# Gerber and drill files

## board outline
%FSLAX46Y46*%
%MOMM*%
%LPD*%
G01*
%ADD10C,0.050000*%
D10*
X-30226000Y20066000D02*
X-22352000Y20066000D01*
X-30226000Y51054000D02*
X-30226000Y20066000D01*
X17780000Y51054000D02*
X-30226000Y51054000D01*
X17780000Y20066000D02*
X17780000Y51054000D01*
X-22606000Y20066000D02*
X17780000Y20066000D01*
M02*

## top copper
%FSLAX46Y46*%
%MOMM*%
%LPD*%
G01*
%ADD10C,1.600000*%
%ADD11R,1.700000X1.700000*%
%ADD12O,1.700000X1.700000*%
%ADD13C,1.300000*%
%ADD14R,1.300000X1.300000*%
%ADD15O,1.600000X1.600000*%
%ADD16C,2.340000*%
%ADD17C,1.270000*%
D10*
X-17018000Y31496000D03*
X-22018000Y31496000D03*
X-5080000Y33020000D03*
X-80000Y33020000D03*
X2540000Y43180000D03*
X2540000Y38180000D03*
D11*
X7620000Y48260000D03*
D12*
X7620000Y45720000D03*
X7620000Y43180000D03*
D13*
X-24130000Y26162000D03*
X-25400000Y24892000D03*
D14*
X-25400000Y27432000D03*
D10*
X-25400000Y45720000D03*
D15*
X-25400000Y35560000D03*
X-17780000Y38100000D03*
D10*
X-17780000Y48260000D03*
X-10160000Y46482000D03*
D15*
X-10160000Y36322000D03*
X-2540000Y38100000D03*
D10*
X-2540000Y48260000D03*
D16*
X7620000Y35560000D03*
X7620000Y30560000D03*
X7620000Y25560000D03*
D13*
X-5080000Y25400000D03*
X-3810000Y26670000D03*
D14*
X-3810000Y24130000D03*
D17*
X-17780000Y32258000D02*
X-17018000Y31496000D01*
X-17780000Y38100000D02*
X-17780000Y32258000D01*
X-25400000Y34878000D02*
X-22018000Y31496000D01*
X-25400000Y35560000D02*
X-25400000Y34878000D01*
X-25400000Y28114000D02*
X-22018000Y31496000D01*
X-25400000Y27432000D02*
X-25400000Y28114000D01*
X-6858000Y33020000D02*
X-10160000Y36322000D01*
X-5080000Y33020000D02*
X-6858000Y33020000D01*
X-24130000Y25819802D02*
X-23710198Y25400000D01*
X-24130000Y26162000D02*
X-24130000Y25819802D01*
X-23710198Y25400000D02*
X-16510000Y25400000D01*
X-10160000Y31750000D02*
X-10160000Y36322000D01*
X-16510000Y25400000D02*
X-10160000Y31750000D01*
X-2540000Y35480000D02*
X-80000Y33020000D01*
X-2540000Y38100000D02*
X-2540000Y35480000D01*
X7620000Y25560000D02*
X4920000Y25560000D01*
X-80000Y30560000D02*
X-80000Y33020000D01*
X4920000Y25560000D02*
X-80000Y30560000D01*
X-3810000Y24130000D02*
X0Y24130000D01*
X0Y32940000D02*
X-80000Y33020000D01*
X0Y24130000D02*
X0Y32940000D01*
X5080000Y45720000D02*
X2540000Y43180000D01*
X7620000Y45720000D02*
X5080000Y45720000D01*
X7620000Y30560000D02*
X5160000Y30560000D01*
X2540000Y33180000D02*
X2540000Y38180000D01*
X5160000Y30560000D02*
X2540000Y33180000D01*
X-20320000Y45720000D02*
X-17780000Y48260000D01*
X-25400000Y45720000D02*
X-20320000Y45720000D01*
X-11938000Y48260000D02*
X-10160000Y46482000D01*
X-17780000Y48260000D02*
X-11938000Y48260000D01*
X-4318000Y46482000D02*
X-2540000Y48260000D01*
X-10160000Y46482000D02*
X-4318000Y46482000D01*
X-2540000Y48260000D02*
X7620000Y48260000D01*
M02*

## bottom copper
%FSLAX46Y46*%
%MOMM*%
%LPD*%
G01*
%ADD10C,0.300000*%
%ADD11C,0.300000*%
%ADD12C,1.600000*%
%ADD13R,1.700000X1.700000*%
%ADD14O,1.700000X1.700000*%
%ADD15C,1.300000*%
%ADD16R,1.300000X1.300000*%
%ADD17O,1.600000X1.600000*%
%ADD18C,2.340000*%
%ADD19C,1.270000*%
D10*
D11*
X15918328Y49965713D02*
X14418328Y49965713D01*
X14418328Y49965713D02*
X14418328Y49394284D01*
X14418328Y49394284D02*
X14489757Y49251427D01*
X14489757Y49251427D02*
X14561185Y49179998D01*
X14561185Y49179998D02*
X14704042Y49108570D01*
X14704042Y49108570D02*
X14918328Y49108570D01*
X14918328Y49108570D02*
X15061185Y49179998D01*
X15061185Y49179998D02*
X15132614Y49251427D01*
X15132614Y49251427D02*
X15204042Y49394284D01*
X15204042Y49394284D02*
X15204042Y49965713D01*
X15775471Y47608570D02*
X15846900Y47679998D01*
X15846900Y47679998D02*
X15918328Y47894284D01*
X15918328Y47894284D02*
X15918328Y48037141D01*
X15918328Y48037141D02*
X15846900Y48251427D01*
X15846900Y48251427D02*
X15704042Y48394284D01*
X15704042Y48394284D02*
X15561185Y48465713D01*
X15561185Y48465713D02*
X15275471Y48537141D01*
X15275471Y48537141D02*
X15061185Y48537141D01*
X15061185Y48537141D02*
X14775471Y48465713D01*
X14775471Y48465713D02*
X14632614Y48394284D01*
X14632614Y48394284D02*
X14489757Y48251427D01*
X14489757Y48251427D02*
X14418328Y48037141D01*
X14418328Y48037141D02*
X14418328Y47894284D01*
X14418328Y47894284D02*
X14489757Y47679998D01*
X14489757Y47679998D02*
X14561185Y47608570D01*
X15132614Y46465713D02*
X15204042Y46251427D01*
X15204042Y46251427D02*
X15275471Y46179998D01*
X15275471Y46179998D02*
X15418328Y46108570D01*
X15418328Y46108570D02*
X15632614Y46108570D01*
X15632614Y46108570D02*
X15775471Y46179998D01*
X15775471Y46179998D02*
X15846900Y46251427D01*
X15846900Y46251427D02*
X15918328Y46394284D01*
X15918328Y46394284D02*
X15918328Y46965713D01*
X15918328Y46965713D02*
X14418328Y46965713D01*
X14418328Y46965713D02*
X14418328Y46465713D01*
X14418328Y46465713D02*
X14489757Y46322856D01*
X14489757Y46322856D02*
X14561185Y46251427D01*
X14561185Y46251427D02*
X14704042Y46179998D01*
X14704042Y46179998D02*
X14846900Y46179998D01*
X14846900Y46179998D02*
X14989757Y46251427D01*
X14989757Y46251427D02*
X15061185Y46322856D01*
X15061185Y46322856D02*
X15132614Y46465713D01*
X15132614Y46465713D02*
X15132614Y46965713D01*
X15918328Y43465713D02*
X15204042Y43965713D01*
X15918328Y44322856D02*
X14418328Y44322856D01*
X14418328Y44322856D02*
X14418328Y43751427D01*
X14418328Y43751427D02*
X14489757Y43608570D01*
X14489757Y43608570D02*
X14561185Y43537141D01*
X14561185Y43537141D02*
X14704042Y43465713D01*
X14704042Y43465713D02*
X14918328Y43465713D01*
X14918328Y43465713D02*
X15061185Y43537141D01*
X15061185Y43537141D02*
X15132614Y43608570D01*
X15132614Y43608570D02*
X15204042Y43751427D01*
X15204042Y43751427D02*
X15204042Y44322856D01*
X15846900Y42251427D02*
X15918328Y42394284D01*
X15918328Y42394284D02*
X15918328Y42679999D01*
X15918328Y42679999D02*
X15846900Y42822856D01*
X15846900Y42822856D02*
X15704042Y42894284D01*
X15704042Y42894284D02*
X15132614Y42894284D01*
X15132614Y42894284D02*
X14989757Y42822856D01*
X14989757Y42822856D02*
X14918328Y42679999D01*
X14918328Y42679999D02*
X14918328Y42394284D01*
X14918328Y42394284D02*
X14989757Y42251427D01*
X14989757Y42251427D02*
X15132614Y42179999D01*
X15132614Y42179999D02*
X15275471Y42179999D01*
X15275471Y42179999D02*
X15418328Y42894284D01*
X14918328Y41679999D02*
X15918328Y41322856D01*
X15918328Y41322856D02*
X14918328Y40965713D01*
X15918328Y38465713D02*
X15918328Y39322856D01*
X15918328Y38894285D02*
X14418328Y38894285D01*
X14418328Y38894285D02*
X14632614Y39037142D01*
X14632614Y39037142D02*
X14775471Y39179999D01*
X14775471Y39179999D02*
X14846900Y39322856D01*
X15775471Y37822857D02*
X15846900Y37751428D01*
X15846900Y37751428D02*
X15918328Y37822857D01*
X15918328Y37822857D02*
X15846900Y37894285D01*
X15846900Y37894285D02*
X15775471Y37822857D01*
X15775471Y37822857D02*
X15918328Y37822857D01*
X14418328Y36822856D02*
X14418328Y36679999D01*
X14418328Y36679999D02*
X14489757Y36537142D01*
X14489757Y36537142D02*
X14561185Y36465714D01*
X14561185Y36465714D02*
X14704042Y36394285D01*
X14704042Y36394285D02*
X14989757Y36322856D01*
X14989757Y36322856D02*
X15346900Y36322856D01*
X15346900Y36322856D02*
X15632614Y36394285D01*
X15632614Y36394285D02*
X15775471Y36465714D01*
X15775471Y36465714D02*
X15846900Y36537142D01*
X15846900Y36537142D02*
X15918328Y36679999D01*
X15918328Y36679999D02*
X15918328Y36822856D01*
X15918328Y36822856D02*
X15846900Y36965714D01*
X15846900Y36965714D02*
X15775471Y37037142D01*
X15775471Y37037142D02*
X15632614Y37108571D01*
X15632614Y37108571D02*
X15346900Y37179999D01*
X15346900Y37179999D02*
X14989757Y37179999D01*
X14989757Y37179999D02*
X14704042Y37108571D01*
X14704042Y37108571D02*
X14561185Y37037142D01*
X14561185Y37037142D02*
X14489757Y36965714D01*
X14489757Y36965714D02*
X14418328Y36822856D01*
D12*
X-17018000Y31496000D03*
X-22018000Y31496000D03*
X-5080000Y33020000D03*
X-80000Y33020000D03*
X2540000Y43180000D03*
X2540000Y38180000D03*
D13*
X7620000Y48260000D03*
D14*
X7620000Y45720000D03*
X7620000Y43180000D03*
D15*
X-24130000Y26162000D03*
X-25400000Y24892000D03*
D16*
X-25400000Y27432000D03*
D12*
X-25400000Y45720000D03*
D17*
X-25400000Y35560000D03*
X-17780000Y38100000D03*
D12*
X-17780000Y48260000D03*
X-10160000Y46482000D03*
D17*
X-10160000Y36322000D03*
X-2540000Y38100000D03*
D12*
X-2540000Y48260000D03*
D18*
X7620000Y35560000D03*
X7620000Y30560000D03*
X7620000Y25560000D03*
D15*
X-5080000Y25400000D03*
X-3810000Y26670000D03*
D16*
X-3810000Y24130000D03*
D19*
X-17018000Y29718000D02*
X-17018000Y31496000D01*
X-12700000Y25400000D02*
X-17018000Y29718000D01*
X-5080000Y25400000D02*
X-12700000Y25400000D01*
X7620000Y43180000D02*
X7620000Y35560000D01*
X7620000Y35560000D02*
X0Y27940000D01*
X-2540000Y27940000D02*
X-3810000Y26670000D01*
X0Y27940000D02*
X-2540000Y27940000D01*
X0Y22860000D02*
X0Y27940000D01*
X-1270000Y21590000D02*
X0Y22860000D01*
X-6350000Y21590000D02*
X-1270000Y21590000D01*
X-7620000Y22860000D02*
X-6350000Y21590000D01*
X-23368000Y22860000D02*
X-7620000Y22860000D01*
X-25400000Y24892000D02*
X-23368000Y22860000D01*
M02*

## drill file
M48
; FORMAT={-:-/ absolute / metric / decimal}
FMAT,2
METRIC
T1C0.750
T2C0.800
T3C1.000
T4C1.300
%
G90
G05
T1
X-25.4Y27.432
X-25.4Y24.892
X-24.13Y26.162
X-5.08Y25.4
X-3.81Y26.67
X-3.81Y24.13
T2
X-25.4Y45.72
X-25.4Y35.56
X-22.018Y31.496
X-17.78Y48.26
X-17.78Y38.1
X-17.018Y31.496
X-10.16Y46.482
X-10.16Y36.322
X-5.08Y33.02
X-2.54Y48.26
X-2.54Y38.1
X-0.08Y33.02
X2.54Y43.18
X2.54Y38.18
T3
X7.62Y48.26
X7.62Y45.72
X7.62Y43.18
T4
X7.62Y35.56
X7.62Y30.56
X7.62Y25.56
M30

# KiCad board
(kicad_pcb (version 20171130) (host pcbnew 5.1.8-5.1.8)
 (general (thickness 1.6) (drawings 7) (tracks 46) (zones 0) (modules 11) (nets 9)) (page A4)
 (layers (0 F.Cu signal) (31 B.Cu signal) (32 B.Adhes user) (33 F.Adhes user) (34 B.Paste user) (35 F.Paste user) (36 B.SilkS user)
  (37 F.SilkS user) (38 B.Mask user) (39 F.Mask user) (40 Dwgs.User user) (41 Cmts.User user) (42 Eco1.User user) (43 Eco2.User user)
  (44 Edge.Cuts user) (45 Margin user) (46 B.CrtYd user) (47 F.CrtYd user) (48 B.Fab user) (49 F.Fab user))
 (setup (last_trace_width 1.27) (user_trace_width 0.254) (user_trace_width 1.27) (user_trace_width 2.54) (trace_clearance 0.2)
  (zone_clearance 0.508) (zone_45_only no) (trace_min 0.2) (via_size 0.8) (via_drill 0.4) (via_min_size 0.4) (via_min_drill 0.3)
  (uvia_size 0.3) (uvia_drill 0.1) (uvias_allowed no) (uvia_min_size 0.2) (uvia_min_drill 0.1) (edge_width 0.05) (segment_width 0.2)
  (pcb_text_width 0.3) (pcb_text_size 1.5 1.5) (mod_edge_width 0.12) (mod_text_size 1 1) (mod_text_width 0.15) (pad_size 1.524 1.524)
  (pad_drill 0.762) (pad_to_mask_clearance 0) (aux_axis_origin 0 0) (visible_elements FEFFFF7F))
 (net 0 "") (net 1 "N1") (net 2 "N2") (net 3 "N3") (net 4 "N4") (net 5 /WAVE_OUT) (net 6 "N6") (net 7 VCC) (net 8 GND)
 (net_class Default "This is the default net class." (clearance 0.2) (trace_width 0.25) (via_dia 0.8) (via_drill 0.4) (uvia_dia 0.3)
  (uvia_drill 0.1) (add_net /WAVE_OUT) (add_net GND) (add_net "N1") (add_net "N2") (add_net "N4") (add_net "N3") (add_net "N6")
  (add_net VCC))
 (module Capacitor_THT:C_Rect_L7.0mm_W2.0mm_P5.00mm (layer F.Cu) (at -17.018 -31.496 180)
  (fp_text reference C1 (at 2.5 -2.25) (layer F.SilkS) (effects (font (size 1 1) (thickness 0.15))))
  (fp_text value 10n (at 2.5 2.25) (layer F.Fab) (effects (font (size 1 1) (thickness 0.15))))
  (pad 1 thru_hole circle (at 0 0 180) (size 1.6 1.6) (drill 0.8) (layers *.Cu *.Mask) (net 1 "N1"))
  (pad 2 thru_hole circle (at 5 0 180) (size 1.6 1.6) (drill 0.8) (layers *.Cu *.Mask) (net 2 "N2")))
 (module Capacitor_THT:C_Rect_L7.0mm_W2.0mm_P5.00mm (layer F.Cu) (at -0.08 -33.02 180)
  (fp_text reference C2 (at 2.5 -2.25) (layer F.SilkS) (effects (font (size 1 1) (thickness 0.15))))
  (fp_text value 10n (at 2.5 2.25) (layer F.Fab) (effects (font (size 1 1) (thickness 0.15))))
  (pad 2 thru_hole circle (at 5 0 180) (size 1.6 1.6) (drill 0.8) (layers *.Cu *.Mask) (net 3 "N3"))
  (pad 1 thru_hole circle (at 0 0 180) (size 1.6 1.6) (drill 0.8) (layers *.Cu *.Mask) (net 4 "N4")))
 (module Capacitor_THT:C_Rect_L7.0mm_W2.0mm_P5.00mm (layer F.Cu) (at 2.54 -43.18 270)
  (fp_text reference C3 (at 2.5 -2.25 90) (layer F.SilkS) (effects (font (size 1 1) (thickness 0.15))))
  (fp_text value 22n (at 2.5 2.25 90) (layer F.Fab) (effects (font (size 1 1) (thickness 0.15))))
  (pad 1 thru_hole circle (at 0 0 270) (size 1.6 1.6) (drill 0.8) (layers *.Cu *.Mask) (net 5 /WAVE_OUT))
  (pad 2 thru_hole circle (at 5 0 270) (size 1.6 1.6) (drill 0.8) (layers *.Cu *.Mask) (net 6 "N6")))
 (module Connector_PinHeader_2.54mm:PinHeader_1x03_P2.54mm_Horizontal (layer F.Cu) (at 7.62 -48.26)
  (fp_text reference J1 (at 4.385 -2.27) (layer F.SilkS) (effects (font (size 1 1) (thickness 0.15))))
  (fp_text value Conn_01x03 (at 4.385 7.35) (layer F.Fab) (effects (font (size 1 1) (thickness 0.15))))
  (pad 1 thru_hole rect (at 0 0) (size 1.7 1.7) (drill 1) (layers *.Cu *.Mask) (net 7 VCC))
  (pad 2 thru_hole oval (at 0 2.54) (size 1.7 1.7) (drill 1) (layers *.Cu *.Mask) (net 5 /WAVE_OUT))
  (pad 3 thru_hole oval (at 0 5.08) (size 1.7 1.7) (drill 1) (layers *.Cu *.Mask) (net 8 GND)))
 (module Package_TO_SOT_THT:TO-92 (layer F.Cu) (at -25.4 -27.432 270)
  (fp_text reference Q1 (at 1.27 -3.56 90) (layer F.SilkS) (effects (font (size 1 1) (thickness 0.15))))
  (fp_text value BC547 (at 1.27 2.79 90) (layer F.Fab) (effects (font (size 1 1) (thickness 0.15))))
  (pad 2 thru_hole circle (at 1.27 -1.27 270) (size 1.3 1.3) (drill 0.75) (layers *.Cu *.Mask) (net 3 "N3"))
  (pad 3 thru_hole circle (at 2.54 0 270) (size 1.3 1.3) (drill 0.75) (layers *.Cu *.Mask) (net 8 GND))
  (pad 1 thru_hole rect (at 0 0 270) (size 1.3 1.3) (drill 0.75) (layers *.Cu *.Mask) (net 2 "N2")))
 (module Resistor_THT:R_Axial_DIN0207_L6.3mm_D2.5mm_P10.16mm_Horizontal (layer F.Cu) (at -25.4 -45.72 270)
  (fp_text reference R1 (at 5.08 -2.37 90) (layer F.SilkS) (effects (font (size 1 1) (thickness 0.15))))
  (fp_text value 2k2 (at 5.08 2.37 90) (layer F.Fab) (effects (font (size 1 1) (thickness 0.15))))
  (pad 1 thru_hole circle (at 0 0 270) (size 1.6 1.6) (drill 0.8) (layers *.Cu *.Mask) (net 7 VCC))
  (pad 2 thru_hole oval (at 10.16 0 270) (size 1.6 1.6) (drill 0.8) (layers *.Cu *.Mask) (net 2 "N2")))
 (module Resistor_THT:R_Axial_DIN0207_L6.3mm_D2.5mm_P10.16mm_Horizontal (layer F.Cu) (at -17.78 -48.26 270)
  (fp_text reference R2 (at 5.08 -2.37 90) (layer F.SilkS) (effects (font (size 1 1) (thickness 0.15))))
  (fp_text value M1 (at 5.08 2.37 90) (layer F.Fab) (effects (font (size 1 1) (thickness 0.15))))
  (pad 2 thru_hole oval (at 10.16 0 270) (size 1.6 1.6) (drill 0.8) (layers *.Cu *.Mask) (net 1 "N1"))
  (pad 1 thru_hole circle (at 0 0 270) (size 1.6 1.6) (drill 0.8) (layers *.Cu *.Mask) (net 7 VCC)))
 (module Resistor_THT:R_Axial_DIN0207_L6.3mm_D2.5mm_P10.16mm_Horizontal (layer F.Cu) (at -10.16 -46.482 270)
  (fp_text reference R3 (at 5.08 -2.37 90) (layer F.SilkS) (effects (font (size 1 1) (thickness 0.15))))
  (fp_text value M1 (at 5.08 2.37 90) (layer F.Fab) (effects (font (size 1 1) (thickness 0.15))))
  (pad 1 thru_hole circle (at 0 0 270) (size 1.6 1.6) (drill 0.8) (layers *.Cu *.Mask) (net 7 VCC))
  (pad 2 thru_hole oval (at 10.16 0 270) (size 1.6 1.6) (drill 0.8) (layers *.Cu *.Mask) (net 3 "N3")))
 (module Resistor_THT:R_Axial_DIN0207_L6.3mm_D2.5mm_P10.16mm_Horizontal (layer F.Cu) (at -2.54 -48.26 270)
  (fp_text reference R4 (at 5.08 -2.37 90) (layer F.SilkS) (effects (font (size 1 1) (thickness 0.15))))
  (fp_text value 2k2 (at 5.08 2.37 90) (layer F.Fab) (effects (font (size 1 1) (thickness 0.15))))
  (pad 2 thru_hole oval (at 10.16 0 270) (size 1.6 1.6) (drill 0.8) (layers *.Cu *.Mask) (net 4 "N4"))
  (pad 1 thru_hole circle (at 0 0 270) (size 1.6 1.6) (drill 0.8) (layers *.Cu *.Mask) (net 7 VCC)))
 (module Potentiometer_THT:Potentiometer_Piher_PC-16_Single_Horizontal (layer F.Cu) (at 7.62 -25.56)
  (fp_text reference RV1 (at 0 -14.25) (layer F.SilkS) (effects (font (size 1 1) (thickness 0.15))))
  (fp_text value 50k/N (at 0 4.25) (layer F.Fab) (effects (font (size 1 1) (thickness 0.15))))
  (pad 3 thru_hole circle (at 0 -10) (size 2.34 2.34) (drill 1.3) (layers *.Cu *.Mask) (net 8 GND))
  (pad 2 thru_hole circle (at 0 -5) (size 2.34 2.34) (drill 1.3) (layers *.Cu *.Mask) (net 6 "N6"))
  (pad 1 thru_hole circle (at 0 0) (size 2.34 2.34) (drill 1.3) (layers *.Cu *.Mask) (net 4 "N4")))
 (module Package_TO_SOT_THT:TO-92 (layer F.Cu) (at -3.81 -24.13 90)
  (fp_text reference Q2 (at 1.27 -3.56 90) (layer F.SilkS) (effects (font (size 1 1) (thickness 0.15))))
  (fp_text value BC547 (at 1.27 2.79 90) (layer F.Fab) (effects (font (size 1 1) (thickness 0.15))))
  (pad 2 thru_hole circle (at 1.27 -1.27 90) (size 1.3 1.3) (drill 0.75) (layers *.Cu *.Mask) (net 1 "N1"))
  (pad 3 thru_hole circle (at 2.54 0 90) (size 1.3 1.3) (drill 0.75) (layers *.Cu *.Mask) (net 8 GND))
  (pad 1 thru_hole rect (at 0 0 90) (size 1.3 1.3) (drill 0.75) (layers *.Cu *.Mask) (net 4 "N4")))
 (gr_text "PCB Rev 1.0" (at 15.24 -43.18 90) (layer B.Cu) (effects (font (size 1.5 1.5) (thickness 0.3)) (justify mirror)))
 (gr_line (start -30.226 -20.066) (end -22.352 -20.066) (layer Edge.Cuts) (width 0.05))
 (gr_line (start -30.226 -51.054) (end -30.226 -20.066) (layer Edge.Cuts) (width 0.05))
 (gr_line (start 17.78 -51.054) (end -30.226 -51.054) (layer Edge.Cuts) (width 0.05))
 (gr_line (start 17.78 -20.066) (end 17.78 -51.054) (layer Edge.Cuts) (width 0.05))
 (gr_line (start -22.606 -20.066) (end 17.78 -20.066) (layer Edge.Cuts) (width 0.05))
 (segment (start -17.78 -32.258) (end -17.018 -31.496) (width 1.27) (layer F.Cu) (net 1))
 (segment (start -17.78 -38.1) (end -17.78 -32.258) (width 1.27) (layer F.Cu) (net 1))
 (segment (start -17.018 -29.718) (end -17.018 -31.496) (width 1.27) (layer B.Cu) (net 1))
 (segment (start -12.7 -25.4) (end -17.018 -29.718) (width 1.27) (layer B.Cu) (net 1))
 (segment (start -5.08 -25.4) (end -12.7 -25.4) (width 1.27) (layer B.Cu) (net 1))
 (segment (start -25.4 -34.878) (end -22.018 -31.496) (width 1.27) (layer F.Cu) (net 2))
 (segment (start -25.4 -35.56) (end -25.4 -34.878) (width 1.27) (layer F.Cu) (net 2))
 (segment (start -25.4 -28.114) (end -22.018 -31.496) (width 1.27) (layer F.Cu) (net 2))
 (segment (start -25.4 -27.432) (end -25.4 -28.114) (width 1.27) (layer F.Cu) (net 2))
 (segment (start -6.858 -33.02) (end -10.16 -36.322) (width 1.27) (layer F.Cu) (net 3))
 (segment (start -5.08 -33.02) (end -6.858 -33.02) (width 1.27) (layer F.Cu) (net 3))
 (segment (start -24.13 -25.819802) (end -23.710198 -25.4) (width 1.27) (layer F.Cu) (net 3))
 (segment (start -24.13 -26.162) (end -24.13 -25.819802) (width 1.27) (layer F.Cu) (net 3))
 (segment (start -23.710198 -25.4) (end -16.51 -25.4) (width 1.27) (layer F.Cu) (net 3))
 (segment (start -10.16 -31.75) (end -10.16 -36.322) (width 1.27) (layer F.Cu) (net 3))
 (segment (start -16.51 -25.4) (end -10.16 -31.75) (width 1.27) (layer F.Cu) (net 3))
 (segment (start -2.54 -35.48) (end -0.08 -33.02) (width 1.27) (layer F.Cu) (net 4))
 (segment (start -2.54 -38.1) (end -2.54 -35.48) (width 1.27) (layer F.Cu) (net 4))
 (segment (start 7.62 -25.56) (end 4.92 -25.56) (width 1.27) (layer F.Cu) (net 4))
 (segment (start -0.08 -30.56) (end -0.08 -33.02) (width 1.27) (layer F.Cu) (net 4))
 (segment (start 4.92 -25.56) (end -0.08 -30.56) (width 1.27) (layer F.Cu) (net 4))
 (segment (start -3.81 -24.13) (end 0 -24.13) (width 1.27) (layer F.Cu) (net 4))
 (segment (start 0 -32.94) (end -0.08 -33.02) (width 1.27) (layer F.Cu) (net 4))
 (segment (start 0 -24.13) (end 0 -32.94) (width 1.27) (layer F.Cu) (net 4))
 (segment (start 5.08 -45.72) (end 2.54 -43.18) (width 1.27) (layer F.Cu) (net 5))
 (segment (start 7.62 -45.72) (end 5.08 -45.72) (width 1.27) (layer F.Cu) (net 5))
 (segment (start 7.62 -30.56) (end 5.16 -30.56) (width 1.27) (layer F.Cu) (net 6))
 (segment (start 2.54 -33.18) (end 2.54 -38.18) (width 1.27) (layer F.Cu) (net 6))
 (segment (start 5.16 -30.56) (end 2.54 -33.18) (width 1.27) (layer F.Cu) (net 6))
 (segment (start -20.32 -45.72) (end -17.78 -48.26) (width 1.27) (layer F.Cu) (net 7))
 (segment (start -25.4 -45.72) (end -20.32 -45.72) (width 1.27) (layer F.Cu) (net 7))
 (segment (start -11.938 -48.26) (end -10.16 -46.482) (width 1.27) (layer F.Cu) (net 7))
 (segment (start -17.78 -48.26) (end -11.938 -48.26) (width 1.27) (layer F.Cu) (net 7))
 (segment (start -4.318 -46.482) (end -2.54 -48.26) (width 1.27) (layer F.Cu) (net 7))
 (segment (start -10.16 -46.482) (end -4.318 -46.482) (width 1.27) (layer F.Cu) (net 7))
 (segment (start -2.54 -48.26) (end 7.62 -48.26) (width 1.27) (layer F.Cu) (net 7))
 (segment (start 7.62 -43.18) (end 7.62 -35.56) (width 1.27) (layer B.Cu) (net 8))
 (segment (start 7.62 -35.56) (end 0 -27.94) (width 1.27) (layer B.Cu) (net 8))
 (segment (start -2.54 -27.94) (end -3.81 -26.67) (width 1.27) (layer B.Cu) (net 8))
 (segment (start 0 -27.94) (end -2.54 -27.94) (width 1.27) (layer B.Cu) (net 8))
 (segment (start 0 -22.86) (end 0 -27.94) (width 1.27) (layer B.Cu) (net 8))
 (segment (start -1.27 -21.59) (end 0 -22.86) (width 1.27) (layer B.Cu) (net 8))
 (segment (start -6.35 -21.59) (end -1.27 -21.59) (width 1.27) (layer B.Cu) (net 8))
 (segment (start -7.62 -22.86) (end -6.35 -21.59) (width 1.27) (layer B.Cu) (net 8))
 (segment (start -23.368 -22.86) (end -7.62 -22.86) (width 1.27) (layer B.Cu) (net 8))
 (segment (start -25.4 -24.892) (end -23.368 -22.86) (width 1.27) (layer B.Cu) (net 8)))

